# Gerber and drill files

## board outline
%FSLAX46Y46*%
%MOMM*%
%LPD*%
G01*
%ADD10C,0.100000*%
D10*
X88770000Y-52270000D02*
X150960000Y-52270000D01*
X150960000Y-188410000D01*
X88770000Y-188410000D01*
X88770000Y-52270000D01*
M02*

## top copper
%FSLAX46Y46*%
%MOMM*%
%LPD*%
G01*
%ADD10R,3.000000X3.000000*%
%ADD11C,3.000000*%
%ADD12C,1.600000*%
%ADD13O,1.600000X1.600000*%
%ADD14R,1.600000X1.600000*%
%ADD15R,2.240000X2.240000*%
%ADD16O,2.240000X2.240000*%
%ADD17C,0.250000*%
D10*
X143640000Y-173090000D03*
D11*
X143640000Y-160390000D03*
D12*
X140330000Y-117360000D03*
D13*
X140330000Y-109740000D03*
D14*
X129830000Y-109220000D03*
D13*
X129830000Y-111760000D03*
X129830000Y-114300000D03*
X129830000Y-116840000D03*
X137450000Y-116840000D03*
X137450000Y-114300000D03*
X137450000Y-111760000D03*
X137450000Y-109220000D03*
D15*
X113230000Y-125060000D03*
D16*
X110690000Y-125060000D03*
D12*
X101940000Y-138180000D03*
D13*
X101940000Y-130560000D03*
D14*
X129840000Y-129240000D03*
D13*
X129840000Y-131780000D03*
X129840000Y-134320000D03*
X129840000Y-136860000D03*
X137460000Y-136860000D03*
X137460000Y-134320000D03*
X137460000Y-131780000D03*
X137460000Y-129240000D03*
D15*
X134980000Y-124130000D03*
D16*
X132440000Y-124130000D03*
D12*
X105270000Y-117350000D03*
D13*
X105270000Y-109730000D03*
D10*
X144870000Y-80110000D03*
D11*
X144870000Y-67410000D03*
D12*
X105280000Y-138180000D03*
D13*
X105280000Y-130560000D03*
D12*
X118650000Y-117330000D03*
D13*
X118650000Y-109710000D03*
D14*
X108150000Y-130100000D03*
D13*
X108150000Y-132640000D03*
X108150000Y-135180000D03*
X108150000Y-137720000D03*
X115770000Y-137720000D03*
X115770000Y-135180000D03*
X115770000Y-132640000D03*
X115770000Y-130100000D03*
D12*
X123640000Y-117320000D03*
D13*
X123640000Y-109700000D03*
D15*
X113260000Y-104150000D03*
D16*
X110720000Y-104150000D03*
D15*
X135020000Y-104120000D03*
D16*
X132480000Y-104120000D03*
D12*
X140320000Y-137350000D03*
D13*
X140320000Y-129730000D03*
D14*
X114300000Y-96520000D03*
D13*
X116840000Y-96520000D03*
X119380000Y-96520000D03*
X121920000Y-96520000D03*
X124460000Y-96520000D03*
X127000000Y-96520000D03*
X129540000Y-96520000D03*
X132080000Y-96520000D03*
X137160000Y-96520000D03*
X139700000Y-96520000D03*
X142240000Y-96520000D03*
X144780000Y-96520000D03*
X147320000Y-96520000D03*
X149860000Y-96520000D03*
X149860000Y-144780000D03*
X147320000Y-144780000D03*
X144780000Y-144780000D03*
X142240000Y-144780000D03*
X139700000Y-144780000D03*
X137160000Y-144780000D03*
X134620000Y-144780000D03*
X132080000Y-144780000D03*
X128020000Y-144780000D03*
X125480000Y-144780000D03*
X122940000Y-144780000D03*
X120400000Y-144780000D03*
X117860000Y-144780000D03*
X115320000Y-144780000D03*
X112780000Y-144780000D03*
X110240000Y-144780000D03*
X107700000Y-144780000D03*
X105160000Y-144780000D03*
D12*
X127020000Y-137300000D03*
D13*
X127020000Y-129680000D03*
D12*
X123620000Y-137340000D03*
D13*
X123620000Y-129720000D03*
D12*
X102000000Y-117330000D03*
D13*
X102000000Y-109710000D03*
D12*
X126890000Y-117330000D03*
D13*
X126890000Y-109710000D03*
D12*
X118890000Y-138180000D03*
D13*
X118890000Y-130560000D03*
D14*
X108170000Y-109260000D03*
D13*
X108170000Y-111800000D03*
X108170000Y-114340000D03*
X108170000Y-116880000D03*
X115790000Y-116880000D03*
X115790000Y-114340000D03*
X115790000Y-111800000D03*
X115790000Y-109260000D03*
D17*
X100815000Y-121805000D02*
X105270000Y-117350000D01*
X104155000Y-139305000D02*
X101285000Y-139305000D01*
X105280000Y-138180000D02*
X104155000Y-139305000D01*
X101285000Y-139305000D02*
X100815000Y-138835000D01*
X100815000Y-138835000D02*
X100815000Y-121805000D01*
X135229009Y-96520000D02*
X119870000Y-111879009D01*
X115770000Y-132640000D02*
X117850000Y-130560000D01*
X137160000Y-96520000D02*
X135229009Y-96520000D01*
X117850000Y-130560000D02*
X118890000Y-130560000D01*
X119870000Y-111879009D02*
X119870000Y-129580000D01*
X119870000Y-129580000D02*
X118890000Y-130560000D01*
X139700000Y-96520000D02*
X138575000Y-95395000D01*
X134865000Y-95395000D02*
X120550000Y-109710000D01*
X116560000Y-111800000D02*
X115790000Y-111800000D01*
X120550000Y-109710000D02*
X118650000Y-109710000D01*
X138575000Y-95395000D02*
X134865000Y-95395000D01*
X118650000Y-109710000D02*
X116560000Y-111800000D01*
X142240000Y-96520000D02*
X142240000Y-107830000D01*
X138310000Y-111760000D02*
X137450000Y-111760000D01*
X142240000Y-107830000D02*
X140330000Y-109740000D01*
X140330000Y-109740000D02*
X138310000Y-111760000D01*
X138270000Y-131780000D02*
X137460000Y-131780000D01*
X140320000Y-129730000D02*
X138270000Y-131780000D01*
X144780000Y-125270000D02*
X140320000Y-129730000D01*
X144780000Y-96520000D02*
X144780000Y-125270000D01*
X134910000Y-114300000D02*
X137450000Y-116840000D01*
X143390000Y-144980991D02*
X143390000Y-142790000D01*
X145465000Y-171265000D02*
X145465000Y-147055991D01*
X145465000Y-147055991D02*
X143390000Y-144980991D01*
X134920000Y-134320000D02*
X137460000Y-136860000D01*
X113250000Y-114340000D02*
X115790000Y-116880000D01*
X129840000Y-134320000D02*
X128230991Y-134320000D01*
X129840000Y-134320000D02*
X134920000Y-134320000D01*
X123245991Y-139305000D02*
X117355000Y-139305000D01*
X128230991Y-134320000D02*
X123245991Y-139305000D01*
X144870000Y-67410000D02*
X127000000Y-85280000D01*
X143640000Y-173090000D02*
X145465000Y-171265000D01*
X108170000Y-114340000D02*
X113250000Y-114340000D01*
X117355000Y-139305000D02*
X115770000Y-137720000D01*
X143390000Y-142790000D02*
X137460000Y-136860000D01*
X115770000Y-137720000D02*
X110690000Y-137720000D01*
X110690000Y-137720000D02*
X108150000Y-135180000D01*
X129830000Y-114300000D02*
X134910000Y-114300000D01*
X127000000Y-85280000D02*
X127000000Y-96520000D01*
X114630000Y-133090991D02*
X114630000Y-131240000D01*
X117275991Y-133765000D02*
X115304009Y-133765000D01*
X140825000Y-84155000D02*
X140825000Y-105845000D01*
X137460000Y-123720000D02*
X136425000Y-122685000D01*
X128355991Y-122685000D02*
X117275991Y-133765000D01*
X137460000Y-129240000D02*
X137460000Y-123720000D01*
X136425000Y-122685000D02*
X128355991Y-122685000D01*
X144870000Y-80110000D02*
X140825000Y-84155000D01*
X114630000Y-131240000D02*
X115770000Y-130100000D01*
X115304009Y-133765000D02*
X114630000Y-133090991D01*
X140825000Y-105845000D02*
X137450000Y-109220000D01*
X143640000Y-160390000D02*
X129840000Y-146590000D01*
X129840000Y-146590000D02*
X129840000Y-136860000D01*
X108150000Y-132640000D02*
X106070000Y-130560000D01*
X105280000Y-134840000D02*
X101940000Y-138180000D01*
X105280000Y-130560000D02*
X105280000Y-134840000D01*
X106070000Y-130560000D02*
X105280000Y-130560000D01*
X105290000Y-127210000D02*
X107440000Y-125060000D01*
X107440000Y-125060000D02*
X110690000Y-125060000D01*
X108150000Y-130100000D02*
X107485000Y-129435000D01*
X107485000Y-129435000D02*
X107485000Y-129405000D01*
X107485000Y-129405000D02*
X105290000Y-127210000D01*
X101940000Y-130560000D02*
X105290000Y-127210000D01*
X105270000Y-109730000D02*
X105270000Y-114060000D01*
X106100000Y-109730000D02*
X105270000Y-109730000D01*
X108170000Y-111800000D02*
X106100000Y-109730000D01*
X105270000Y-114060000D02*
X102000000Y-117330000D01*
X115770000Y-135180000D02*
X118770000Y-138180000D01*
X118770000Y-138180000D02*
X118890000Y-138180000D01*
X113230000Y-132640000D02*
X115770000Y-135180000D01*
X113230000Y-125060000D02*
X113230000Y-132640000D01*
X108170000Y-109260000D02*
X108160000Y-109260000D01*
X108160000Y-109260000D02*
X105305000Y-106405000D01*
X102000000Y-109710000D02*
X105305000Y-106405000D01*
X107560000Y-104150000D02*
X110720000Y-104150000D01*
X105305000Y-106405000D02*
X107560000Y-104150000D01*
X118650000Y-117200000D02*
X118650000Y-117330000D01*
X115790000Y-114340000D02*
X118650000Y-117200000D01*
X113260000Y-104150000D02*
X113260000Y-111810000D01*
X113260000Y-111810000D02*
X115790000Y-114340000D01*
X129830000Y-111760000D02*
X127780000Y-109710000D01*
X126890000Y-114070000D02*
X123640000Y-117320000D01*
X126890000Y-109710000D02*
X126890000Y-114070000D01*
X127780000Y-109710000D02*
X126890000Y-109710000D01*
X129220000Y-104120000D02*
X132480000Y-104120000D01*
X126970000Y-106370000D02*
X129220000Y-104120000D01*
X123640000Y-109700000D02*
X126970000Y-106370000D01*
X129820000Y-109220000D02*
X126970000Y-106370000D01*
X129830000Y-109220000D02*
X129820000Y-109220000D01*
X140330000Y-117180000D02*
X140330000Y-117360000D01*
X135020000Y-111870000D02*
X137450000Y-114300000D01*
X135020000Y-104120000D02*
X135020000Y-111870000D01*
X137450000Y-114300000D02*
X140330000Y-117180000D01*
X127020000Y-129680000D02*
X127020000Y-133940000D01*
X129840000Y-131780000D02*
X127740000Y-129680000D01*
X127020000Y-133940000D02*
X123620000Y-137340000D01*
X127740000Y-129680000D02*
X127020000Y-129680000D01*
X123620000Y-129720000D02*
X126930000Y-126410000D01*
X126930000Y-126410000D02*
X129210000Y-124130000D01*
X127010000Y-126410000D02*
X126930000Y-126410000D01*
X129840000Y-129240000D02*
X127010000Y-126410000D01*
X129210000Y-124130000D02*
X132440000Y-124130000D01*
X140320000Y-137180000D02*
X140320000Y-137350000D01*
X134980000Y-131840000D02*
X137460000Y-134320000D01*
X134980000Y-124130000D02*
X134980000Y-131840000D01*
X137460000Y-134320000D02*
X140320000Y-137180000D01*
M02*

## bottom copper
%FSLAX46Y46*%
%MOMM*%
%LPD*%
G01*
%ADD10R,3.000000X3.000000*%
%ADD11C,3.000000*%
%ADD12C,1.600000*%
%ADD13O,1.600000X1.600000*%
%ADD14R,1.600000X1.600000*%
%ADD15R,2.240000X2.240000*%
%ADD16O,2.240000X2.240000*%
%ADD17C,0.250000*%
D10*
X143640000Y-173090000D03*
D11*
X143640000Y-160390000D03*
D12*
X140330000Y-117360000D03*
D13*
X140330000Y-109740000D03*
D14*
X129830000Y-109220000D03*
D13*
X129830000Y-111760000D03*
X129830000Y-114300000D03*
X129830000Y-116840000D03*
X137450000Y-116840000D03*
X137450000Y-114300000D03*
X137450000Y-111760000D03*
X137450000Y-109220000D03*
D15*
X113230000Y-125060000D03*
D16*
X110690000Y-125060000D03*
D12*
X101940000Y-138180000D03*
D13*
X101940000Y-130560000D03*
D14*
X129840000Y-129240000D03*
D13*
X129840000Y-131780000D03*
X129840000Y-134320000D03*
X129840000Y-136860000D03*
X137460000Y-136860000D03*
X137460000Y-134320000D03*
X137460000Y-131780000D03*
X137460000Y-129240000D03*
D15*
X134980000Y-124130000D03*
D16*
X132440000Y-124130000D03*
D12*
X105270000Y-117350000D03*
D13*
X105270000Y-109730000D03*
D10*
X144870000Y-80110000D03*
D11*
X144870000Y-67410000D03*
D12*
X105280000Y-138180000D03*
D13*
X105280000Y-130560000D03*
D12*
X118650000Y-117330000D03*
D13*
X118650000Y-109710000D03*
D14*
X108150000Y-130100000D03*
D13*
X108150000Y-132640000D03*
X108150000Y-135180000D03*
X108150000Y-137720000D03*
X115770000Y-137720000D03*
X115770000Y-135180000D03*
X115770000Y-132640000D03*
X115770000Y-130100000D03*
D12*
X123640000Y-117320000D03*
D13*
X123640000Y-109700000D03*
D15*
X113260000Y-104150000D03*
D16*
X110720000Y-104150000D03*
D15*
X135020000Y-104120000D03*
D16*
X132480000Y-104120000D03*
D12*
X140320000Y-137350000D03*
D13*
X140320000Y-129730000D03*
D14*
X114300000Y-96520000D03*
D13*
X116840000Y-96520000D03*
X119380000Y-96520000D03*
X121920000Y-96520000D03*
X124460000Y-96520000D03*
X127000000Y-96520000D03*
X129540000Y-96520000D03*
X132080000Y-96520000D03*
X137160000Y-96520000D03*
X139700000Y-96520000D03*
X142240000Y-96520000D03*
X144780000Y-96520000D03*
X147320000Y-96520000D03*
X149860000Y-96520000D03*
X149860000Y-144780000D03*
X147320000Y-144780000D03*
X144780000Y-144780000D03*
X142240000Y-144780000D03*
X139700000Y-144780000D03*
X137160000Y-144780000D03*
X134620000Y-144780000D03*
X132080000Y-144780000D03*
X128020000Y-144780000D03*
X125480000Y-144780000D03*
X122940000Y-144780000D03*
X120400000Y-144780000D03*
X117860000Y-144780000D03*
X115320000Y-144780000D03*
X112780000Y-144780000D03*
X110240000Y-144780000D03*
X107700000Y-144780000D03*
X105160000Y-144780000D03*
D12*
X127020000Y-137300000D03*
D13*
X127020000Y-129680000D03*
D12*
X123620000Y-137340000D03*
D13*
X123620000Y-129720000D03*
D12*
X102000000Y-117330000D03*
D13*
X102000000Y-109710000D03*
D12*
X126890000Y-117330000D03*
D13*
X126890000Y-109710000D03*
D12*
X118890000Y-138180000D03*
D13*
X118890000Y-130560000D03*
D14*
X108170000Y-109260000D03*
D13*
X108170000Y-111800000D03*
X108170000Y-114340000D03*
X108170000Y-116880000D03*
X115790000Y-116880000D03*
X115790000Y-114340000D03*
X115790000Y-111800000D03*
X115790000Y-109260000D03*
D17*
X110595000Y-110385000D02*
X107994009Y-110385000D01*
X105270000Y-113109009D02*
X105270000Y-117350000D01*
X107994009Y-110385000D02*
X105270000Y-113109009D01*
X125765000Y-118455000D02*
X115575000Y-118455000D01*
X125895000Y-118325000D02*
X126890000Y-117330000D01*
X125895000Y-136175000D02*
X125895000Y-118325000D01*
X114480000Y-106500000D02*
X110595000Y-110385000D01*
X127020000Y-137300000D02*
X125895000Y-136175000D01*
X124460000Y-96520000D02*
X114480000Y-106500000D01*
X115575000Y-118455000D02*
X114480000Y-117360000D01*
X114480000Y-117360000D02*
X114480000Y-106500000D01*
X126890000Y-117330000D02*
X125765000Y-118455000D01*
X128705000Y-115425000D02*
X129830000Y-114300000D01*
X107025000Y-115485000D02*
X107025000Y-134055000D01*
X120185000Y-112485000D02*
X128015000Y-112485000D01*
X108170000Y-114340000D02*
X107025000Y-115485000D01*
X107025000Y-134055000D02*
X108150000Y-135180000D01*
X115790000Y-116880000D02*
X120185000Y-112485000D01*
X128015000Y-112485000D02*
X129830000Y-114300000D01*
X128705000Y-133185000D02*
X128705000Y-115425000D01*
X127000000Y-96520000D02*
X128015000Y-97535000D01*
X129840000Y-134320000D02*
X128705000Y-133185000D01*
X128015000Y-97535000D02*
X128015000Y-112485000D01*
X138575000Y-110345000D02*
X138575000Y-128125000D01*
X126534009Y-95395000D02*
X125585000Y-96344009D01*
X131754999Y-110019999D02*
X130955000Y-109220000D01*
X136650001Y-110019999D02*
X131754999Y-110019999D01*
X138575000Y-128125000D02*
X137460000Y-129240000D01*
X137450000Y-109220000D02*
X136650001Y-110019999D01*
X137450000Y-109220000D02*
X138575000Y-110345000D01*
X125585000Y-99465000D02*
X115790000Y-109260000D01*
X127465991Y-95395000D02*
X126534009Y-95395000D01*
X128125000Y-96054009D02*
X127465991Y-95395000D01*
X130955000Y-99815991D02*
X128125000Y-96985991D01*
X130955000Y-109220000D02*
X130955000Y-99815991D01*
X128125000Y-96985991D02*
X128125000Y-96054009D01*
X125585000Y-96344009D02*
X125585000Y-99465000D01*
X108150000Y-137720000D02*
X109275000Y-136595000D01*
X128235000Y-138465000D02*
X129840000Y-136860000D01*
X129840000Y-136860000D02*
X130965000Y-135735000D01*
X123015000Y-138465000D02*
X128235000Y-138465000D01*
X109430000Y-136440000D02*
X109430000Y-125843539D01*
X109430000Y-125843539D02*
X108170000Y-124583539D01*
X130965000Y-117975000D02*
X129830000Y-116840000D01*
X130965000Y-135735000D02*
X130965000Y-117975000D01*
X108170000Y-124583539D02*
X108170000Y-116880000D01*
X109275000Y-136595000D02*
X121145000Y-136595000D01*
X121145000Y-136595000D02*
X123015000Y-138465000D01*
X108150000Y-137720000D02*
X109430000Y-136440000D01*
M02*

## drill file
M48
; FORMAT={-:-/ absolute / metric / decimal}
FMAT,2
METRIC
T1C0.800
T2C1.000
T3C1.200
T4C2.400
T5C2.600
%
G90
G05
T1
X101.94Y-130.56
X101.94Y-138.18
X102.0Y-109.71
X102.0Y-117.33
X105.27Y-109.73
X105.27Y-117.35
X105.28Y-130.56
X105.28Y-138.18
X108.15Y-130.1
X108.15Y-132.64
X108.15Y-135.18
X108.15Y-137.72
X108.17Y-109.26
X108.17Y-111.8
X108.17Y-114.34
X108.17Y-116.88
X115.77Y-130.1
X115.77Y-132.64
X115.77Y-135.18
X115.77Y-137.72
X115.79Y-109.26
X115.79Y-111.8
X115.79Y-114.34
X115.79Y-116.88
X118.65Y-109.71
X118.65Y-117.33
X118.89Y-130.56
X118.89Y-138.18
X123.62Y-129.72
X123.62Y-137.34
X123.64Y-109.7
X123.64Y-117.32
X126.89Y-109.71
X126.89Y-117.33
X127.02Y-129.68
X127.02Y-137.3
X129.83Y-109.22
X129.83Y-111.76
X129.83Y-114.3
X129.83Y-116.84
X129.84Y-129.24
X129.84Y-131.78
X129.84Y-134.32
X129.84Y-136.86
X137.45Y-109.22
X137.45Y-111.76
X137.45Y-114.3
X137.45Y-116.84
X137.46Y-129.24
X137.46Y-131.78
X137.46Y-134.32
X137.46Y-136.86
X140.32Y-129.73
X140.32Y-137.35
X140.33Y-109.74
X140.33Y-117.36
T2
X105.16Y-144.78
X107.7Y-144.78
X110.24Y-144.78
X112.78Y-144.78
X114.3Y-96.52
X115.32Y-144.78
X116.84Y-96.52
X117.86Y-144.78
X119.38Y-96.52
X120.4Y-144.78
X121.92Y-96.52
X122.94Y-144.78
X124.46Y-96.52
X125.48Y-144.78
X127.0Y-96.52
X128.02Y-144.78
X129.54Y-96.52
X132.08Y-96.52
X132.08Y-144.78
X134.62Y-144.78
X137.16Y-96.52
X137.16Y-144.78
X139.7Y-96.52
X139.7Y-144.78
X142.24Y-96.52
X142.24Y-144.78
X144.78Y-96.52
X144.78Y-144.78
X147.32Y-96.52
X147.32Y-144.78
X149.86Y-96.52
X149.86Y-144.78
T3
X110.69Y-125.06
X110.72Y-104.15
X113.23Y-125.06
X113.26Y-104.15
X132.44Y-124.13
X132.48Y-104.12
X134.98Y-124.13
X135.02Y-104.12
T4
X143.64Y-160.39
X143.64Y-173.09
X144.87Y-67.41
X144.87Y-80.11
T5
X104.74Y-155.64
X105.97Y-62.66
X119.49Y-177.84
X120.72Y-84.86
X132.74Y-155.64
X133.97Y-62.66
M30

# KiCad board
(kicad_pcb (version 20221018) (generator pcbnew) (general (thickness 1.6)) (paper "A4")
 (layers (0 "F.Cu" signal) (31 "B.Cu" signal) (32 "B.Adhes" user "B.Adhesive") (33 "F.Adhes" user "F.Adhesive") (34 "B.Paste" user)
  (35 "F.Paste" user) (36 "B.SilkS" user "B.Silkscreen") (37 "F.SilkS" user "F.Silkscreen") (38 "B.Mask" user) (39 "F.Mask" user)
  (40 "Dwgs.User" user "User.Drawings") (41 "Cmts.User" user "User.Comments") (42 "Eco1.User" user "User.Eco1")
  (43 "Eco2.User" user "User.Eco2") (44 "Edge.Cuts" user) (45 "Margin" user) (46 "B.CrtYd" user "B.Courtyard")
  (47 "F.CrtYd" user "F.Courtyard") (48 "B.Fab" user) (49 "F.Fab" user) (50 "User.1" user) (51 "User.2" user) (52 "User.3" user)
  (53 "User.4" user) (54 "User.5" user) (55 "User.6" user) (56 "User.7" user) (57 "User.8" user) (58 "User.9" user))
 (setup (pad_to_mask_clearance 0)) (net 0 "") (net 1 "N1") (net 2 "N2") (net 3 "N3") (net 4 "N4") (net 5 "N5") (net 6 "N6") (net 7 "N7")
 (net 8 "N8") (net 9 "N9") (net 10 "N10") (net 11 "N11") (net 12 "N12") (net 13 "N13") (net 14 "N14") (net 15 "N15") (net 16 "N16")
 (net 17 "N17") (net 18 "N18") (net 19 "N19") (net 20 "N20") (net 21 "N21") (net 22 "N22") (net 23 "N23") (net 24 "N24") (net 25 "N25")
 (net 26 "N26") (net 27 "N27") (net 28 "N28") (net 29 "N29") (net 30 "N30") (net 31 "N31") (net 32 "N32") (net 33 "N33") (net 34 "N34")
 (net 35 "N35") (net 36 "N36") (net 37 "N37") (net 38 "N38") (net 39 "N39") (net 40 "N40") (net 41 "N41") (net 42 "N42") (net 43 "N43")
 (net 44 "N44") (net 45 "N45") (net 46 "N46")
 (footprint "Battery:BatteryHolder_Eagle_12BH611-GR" (layer "F.Cu") (at 143.64 173.09)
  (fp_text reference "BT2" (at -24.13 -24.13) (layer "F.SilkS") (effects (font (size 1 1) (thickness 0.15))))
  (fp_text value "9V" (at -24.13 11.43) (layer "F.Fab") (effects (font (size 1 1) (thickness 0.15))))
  (pad "" np_thru_hole circle (at -38.9 -17.45) (size 2.6 2.6) (drill 2.6) (layers "*.Cu" "*.Mask"))
  (pad "" np_thru_hole circle (at -24.15 4.75) (size 2.6 2.6) (drill 2.6) (layers "*.Cu" "*.Mask"))
  (pad "" np_thru_hole circle (at -10.9 -17.45) (size 2.6 2.6) (drill 2.6) (layers "*.Cu" "*.Mask"))
  (pad "1" thru_hole rect (at 0 0) (size 3 3) (drill 2.4) (layers "*.Cu" "*.Mask") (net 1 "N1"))
  (pad "2" thru_hole circle (at 0 -12.7) (size 3 3) (drill 2.4) (layers "*.Cu" "*.Mask") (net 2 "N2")))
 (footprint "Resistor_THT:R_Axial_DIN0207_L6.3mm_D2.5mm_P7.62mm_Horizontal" (layer "F.Cu") (at 140.33 117.36 90)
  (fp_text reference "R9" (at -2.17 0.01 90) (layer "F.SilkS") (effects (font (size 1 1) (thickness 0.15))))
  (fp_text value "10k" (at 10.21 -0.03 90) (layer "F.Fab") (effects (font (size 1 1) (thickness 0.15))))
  (pad "1" thru_hole circle (at 0 0 90) (size 1.6 1.6) (drill 0.8) (layers "*.Cu" "*.Mask") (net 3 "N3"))
  (pad "2" thru_hole oval (at 7.62 0 90) (size 1.6 1.6) (drill 0.8) (layers "*.Cu" "*.Mask") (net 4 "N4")))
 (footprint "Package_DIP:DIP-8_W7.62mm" (layer "F.Cu") (at 129.83 109.22)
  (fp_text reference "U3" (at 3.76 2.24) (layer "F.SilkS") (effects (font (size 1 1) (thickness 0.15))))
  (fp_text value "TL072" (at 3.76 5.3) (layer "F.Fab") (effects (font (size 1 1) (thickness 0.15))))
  (pad "1" thru_hole rect (at 0 0) (size 1.6 1.6) (drill 0.8) (layers "*.Cu" "*.Mask") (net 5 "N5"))
  (pad "2" thru_hole oval (at 0 2.54) (size 1.6 1.6) (drill 0.8) (layers "*.Cu" "*.Mask") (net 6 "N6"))
  (pad "3" thru_hole oval (at 0 5.08) (size 1.6 1.6) (drill 0.8) (layers "*.Cu" "*.Mask") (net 1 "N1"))
  (pad "4" thru_hole oval (at 0 7.62) (size 1.6 1.6) (drill 0.8) (layers "*.Cu" "*.Mask") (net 2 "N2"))
  (pad "5" thru_hole oval (at 7.62 7.62) (size 1.6 1.6) (drill 0.8) (layers "*.Cu" "*.Mask") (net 1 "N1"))
  (pad "6" thru_hole oval (at 7.62 5.08) (size 1.6 1.6) (drill 0.8) (layers "*.Cu" "*.Mask") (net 3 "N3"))
  (pad "7" thru_hole oval (at 7.62 2.54) (size 1.6 1.6) (drill 0.8) (layers "*.Cu" "*.Mask") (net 4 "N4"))
  (pad "8" thru_hole oval (at 7.62 0) (size 1.6 1.6) (drill 0.8) (layers "*.Cu" "*.Mask") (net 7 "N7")))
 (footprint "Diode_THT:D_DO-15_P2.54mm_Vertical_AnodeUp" (layer "F.Cu") (at 113.23 125.06 180)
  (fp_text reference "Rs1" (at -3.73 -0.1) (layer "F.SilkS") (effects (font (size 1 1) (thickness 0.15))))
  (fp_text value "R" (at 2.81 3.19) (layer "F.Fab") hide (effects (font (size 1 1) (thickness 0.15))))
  (pad "1" thru_hole rect (at 0 0 180) (size 2.24 2.24) (drill 1.2) (layers "*.Cu" "*.Mask") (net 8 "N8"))
  (pad "2" thru_hole oval (at 2.54 0 180) (size 2.24 2.24) (drill 1.2) (layers "*.Cu" "*.Mask") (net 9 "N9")))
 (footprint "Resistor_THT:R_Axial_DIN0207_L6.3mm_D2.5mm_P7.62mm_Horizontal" (layer "F.Cu") (at 101.94 138.18 90)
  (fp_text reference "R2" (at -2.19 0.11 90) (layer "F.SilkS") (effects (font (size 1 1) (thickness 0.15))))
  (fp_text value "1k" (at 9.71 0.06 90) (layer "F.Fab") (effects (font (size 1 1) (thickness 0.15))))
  (pad "1" thru_hole circle (at 0 0 90) (size 1.6 1.6) (drill 0.8) (layers "*.Cu" "*.Mask") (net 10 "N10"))
  (pad "2" thru_hole oval (at 7.62 0 90) (size 1.6 1.6) (drill 0.8) (layers "*.Cu" "*.Mask") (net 9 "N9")))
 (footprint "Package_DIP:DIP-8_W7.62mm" (layer "F.Cu") (at 129.84 129.24)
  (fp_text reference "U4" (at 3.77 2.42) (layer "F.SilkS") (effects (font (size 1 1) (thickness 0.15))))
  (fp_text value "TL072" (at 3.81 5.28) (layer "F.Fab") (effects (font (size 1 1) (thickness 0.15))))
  (pad "1" thru_hole rect (at 0 0) (size 1.6 1.6) (drill 0.8) (layers "*.Cu" "*.Mask") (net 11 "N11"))
  (pad "2" thru_hole oval (at 0 2.54) (size 1.6 1.6) (drill 0.8) (layers "*.Cu" "*.Mask") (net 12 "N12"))
  (pad "3" thru_hole oval (at 0 5.08) (size 1.6 1.6) (drill 0.8) (layers "*.Cu" "*.Mask") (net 1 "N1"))
  (pad "4" thru_hole oval (at 0 7.62) (size 1.6 1.6) (drill 0.8) (layers "*.Cu" "*.Mask") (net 2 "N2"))
  (pad "5" thru_hole oval (at 7.62 7.62) (size 1.6 1.6) (drill 0.8) (layers "*.Cu" "*.Mask") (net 1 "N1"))
  (pad "6" thru_hole oval (at 7.62 5.08) (size 1.6 1.6) (drill 0.8) (layers "*.Cu" "*.Mask") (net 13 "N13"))
  (pad "7" thru_hole oval (at 7.62 2.54) (size 1.6 1.6) (drill 0.8) (layers "*.Cu" "*.Mask") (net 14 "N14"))
  (pad "8" thru_hole oval (at 7.62 0) (size 1.6 1.6) (drill 0.8) (layers "*.Cu" "*.Mask") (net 7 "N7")))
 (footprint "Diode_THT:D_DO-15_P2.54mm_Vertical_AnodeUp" (layer "F.Cu") (at 134.98 124.13 180)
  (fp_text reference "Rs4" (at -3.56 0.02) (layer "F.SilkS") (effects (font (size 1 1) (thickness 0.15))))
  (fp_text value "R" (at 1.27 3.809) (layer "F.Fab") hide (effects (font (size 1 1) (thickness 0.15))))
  (pad "1" thru_hole rect (at 0 0 180) (size 2.24 2.24) (drill 1.2) (layers "*.Cu" "*.Mask") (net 13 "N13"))
  (pad "2" thru_hole oval (at 2.54 0 180) (size 2.24 2.24) (drill 1.2) (layers "*.Cu" "*.Mask") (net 11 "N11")))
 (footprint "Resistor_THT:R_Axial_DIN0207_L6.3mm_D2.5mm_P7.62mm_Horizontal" (layer "F.Cu") (at 105.27 117.35 90)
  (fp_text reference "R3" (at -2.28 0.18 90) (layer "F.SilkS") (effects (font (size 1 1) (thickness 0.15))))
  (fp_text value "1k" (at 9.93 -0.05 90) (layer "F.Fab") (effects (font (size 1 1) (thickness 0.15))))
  (pad "1" thru_hole circle (at 0 0 90) (size 1.6 1.6) (drill 0.8) (layers "*.Cu" "*.Mask") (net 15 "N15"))
  (pad "2" thru_hole oval (at 7.62 0 90) (size 1.6 1.6) (drill 0.8) (layers "*.Cu" "*.Mask") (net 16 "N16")))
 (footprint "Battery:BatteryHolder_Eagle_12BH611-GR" (layer "F.Cu") (at 144.87 80.11)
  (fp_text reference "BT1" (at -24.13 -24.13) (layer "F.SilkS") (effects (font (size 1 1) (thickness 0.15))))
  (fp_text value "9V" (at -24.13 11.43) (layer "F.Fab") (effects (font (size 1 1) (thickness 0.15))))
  (pad "" np_thru_hole circle (at -38.9 -17.45) (size 2.6 2.6) (drill 2.6) (layers "*.Cu" "*.Mask"))
  (pad "" np_thru_hole circle (at -24.15 4.75) (size 2.6 2.6) (drill 2.6) (layers "*.Cu" "*.Mask"))
  (pad "" np_thru_hole circle (at -10.9 -17.45) (size 2.6 2.6) (drill 2.6) (layers "*.Cu" "*.Mask"))
  (pad "1" thru_hole rect (at 0 0) (size 3 3) (drill 2.4) (layers "*.Cu" "*.Mask") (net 7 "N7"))
  (pad "2" thru_hole circle (at 0 -12.7) (size 3 3) (drill 2.4) (layers "*.Cu" "*.Mask") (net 1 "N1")))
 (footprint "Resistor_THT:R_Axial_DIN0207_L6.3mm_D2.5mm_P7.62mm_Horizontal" (layer "F.Cu") (at 105.28 138.18 90)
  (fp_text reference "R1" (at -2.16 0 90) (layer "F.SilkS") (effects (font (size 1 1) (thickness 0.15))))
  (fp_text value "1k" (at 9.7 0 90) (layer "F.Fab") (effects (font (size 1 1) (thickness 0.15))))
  (pad "1" thru_hole circle (at 0 0 90) (size 1.6 1.6) (drill 0.8) (layers "*.Cu" "*.Mask") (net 15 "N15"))
  (pad "2" thru_hole oval (at 7.62 0 90) (size 1.6 1.6) (drill 0.8) (layers "*.Cu" "*.Mask") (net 10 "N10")))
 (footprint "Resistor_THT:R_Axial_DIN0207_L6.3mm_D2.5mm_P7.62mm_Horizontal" (layer "F.Cu") (at 118.65 117.33 90)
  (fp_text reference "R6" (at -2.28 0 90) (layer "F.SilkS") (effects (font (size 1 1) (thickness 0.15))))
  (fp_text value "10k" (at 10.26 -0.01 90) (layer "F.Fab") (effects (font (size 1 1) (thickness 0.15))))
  (pad "1" thru_hole circle (at 0 0 90) (size 1.6 1.6) (drill 0.8) (layers "*.Cu" "*.Mask") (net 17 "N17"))
  (pad "2" thru_hole oval (at 7.62 0 90) (size 1.6 1.6) (drill 0.8) (layers "*.Cu" "*.Mask") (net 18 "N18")))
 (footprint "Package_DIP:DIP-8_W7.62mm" (layer "F.Cu") (at 108.15 130.1)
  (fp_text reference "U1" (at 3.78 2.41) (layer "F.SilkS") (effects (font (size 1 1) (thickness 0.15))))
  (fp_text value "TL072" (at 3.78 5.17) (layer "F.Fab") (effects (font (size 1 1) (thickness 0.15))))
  (pad "1" thru_hole rect (at 0 0) (size 1.6 1.6) (drill 0.8) (layers "*.Cu" "*.Mask") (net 9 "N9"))
  (pad "2" thru_hole oval (at 0 2.54) (size 1.6 1.6) (drill 0.8) (layers "*.Cu" "*.Mask") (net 10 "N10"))
  (pad "3" thru_hole oval (at 0 5.08) (size 1.6 1.6) (drill 0.8) (layers "*.Cu" "*.Mask") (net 1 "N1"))
  (pad "4" thru_hole oval (at 0 7.62) (size 1.6 1.6) (drill 0.8) (layers "*.Cu" "*.Mask") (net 2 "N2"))
  (pad "5" thru_hole oval (at 7.62 7.62) (size 1.6 1.6) (drill 0.8) (layers "*.Cu" "*.Mask") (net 1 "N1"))
  (pad "6" thru_hole oval (at 7.62 5.08) (size 1.6 1.6) (drill 0.8) (layers "*.Cu" "*.Mask") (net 8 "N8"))
  (pad "7" thru_hole oval (at 7.62 2.54) (size 1.6 1.6) (drill 0.8) (layers "*.Cu" "*.Mask") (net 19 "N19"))
  (pad "8" thru_hole oval (at 7.62 0) (size 1.6 1.6) (drill 0.8) (layers "*.Cu" "*.Mask") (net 7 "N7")))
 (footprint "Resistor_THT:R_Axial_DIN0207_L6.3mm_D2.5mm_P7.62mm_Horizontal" (layer "F.Cu") (at 123.64 117.32 90)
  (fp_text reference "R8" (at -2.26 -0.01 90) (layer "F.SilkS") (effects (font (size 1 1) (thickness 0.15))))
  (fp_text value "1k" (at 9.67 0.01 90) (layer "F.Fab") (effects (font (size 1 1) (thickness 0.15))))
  (pad "1" thru_hole circle (at 0 0 90) (size 1.6 1.6) (drill 0.8) (layers "*.Cu" "*.Mask") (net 6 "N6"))
  (pad "2" thru_hole oval (at 7.62 0 90) (size 1.6 1.6) (drill 0.8) (layers "*.Cu" "*.Mask") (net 5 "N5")))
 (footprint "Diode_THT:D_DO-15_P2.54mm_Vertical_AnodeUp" (layer "F.Cu") (at 113.26 104.15 180)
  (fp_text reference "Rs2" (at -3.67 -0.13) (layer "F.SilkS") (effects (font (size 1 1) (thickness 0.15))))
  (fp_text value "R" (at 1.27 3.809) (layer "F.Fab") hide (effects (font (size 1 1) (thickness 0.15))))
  (pad "1" thru_hole rect (at 0 0 180) (size 2.24 2.24) (drill 1.2) (layers "*.Cu" "*.Mask") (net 17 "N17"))
  (pad "2" thru_hole oval (at 2.54 0 180) (size 2.24 2.24) (drill 1.2) (layers "*.Cu" "*.Mask") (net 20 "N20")))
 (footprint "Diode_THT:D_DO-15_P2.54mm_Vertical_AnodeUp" (layer "F.Cu") (at 135.02 104.12 180)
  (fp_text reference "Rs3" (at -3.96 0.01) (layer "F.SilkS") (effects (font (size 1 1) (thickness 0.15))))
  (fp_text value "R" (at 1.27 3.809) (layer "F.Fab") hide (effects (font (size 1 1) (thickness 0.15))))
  (pad "1" thru_hole rect (at 0 0 180) (size 2.24 2.24) (drill 1.2) (layers "*.Cu" "*.Mask") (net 3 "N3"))
  (pad "2" thru_hole oval (at 2.54 0 180) (size 2.24 2.24) (drill 1.2) (layers "*.Cu" "*.Mask") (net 5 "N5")))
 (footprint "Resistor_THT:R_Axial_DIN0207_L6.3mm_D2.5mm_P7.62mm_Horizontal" (layer "F.Cu") (at 140.32 137.35 90)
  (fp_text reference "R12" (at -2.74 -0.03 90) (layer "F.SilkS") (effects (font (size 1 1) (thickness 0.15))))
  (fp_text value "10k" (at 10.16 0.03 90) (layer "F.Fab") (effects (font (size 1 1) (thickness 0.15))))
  (pad "1" thru_hole circle (at 0 0 90) (size 1.6 1.6) (drill 0.8) (layers "*.Cu" "*.Mask") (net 13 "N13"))
  (pad "2" thru_hole oval (at 7.62 0 90) (size 1.6 1.6) (drill 0.8) (layers "*.Cu" "*.Mask") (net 14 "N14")))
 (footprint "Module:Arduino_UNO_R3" (layer "F.Cu") (at 114.3 96.52)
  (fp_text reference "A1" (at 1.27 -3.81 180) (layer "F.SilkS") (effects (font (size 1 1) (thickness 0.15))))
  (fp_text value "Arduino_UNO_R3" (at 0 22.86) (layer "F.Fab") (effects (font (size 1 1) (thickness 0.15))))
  (pad "1" thru_hole rect (at 0 0 90) (size 1.6 1.6) (drill 1) (layers "*.Cu" "*.Mask") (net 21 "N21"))
  (pad "2" thru_hole oval (at 2.54 0 90) (size 1.6 1.6) (drill 1) (layers "*.Cu" "*.Mask") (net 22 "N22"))
  (pad "3" thru_hole oval (at 5.08 0 90) (size 1.6 1.6) (drill 1) (layers "*.Cu" "*.Mask") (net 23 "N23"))
  (pad "4" thru_hole oval (at 7.62 0 90) (size 1.6 1.6) (drill 1) (layers "*.Cu" "*.Mask") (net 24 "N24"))
  (pad "5" thru_hole oval (at 10.16 0 90) (size 1.6 1.6) (drill 1) (layers "*.Cu" "*.Mask") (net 15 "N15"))
  (pad "6" thru_hole oval (at 12.7 0 90) (size 1.6 1.6) (drill 1) (layers "*.Cu" "*.Mask") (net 1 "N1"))
  (pad "7" thru_hole oval (at 15.24 0 90) (size 1.6 1.6) (drill 1) (layers "*.Cu" "*.Mask") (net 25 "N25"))
  (pad "8" thru_hole oval (at 17.78 0 90) (size 1.6 1.6) (drill 1) (layers "*.Cu" "*.Mask") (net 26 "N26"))
  (pad "9" thru_hole oval (at 22.86 0 90) (size 1.6 1.6) (drill 1) (layers "*.Cu" "*.Mask") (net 19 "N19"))
  (pad "10" thru_hole oval (at 25.4 0 90) (size 1.6 1.6) (drill 1) (layers "*.Cu" "*.Mask") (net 18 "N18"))
  (pad "11" thru_hole oval (at 27.94 0 90) (size 1.6 1.6) (drill 1) (layers "*.Cu" "*.Mask") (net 4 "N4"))
  (pad "12" thru_hole oval (at 30.48 0 90) (size 1.6 1.6) (drill 1) (layers "*.Cu" "*.Mask") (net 14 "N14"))
  (pad "13" thru_hole oval (at 33.02 0 90) (size 1.6 1.6) (drill 1) (layers "*.Cu" "*.Mask") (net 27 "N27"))
  (pad "14" thru_hole oval (at 35.56 0 90) (size 1.6 1.6) (drill 1) (layers "*.Cu" "*.Mask") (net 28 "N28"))
  (pad "15" thru_hole oval (at 35.56 48.26 90) (size 1.6 1.6) (drill 1) (layers "*.Cu" "*.Mask") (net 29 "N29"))
  (pad "16" thru_hole oval (at 33.02 48.26 90) (size 1.6 1.6) (drill 1) (layers "*.Cu" "*.Mask") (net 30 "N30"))
  (pad "17" thru_hole oval (at 30.48 48.26 90) (size 1.6 1.6) (drill 1) (layers "*.Cu" "*.Mask") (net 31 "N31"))
  (pad "18" thru_hole oval (at 27.94 48.26 90) (size 1.6 1.6) (drill 1) (layers "*.Cu" "*.Mask") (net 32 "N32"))
  (pad "19" thru_hole oval (at 25.4 48.26 90) (size 1.6 1.6) (drill 1) (layers "*.Cu" "*.Mask") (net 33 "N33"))
  (pad "20" thru_hole oval (at 22.86 48.26 90) (size 1.6 1.6) (drill 1) (layers "*.Cu" "*.Mask") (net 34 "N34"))
  (pad "21" thru_hole oval (at 20.32 48.26 90) (size 1.6 1.6) (drill 1) (layers "*.Cu" "*.Mask") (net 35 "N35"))
  (pad "22" thru_hole oval (at 17.78 48.26 90) (size 1.6 1.6) (drill 1) (layers "*.Cu" "*.Mask") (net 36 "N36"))
  (pad "23" thru_hole oval (at 13.72 48.26 90) (size 1.6 1.6) (drill 1) (layers "*.Cu" "*.Mask") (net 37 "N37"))
  (pad "24" thru_hole oval (at 11.18 48.26 90) (size 1.6 1.6) (drill 1) (layers "*.Cu" "*.Mask") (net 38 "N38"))
  (pad "25" thru_hole oval (at 8.64 48.26 90) (size 1.6 1.6) (drill 1) (layers "*.Cu" "*.Mask") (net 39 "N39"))
  (pad "26" thru_hole oval (at 6.1 48.26 90) (size 1.6 1.6) (drill 1) (layers "*.Cu" "*.Mask") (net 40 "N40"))
  (pad "27" thru_hole oval (at 3.56 48.26 90) (size 1.6 1.6) (drill 1) (layers "*.Cu" "*.Mask") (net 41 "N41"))
  (pad "28" thru_hole oval (at 1.02 48.26 90) (size 1.6 1.6) (drill 1) (layers "*.Cu" "*.Mask") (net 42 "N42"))
  (pad "29" thru_hole oval (at -1.52 48.26 90) (size 1.6 1.6) (drill 1) (layers "*.Cu" "*.Mask") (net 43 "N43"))
  (pad "30" thru_hole oval (at -4.06 48.26 90) (size 1.6 1.6) (drill 1) (layers "*.Cu" "*.Mask") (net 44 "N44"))
  (pad "31" thru_hole oval (at -6.6 48.26 90) (size 1.6 1.6) (drill 1) (layers "*.Cu" "*.Mask") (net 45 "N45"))
  (pad "32" thru_hole oval (at -9.14 48.26 90) (size 1.6 1.6) (drill 1) (layers "*.Cu" "*.Mask") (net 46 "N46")))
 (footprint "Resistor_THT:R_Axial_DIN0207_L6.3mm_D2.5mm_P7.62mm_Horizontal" (layer "F.Cu") (at 127.02 137.3 90)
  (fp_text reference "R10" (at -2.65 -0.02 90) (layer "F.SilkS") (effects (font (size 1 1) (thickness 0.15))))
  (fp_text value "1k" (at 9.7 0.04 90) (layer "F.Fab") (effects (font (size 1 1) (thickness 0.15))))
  (pad "1" thru_hole circle (at 0 0 90) (size 1.6 1.6) (drill 0.8) (layers "*.Cu" "*.Mask") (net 15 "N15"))
  (pad "2" thru_hole oval (at 7.62 0 90) (size 1.6 1.6) (drill 0.8) (layers "*.Cu" "*.Mask") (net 12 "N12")))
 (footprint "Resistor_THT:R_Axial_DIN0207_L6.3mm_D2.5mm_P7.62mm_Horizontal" (layer "F.Cu") (at 123.62 137.34 90)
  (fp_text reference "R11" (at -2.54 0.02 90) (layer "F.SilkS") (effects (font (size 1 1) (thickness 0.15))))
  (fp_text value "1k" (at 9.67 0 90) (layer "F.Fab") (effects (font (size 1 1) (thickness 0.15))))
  (pad "1" thru_hole circle (at 0 0 90) (size 1.6 1.6) (drill 0.8) (layers "*.Cu" "*.Mask") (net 12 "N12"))
  (pad "2" thru_hole oval (at 7.62 0 90) (size 1.6 1.6) (drill 0.8) (layers "*.Cu" "*.Mask") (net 11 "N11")))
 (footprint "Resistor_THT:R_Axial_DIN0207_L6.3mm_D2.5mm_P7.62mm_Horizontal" (layer "F.Cu") (at 102 117.33 90)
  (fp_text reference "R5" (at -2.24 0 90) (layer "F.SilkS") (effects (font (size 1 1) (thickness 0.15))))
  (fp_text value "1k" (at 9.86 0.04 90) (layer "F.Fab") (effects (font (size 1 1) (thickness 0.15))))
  (pad "1" thru_hole circle (at 0 0 90) (size 1.6 1.6) (drill 0.8) (layers "*.Cu" "*.Mask") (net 16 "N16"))
  (pad "2" thru_hole oval (at 7.62 0 90) (size 1.6 1.6) (drill 0.8) (layers "*.Cu" "*.Mask") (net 20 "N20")))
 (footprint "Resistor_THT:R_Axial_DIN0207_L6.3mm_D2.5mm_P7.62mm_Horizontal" (layer "F.Cu") (at 126.89 117.33 90)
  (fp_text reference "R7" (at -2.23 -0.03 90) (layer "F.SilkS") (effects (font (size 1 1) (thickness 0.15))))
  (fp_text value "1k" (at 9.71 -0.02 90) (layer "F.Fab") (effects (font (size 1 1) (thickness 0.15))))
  (pad "1" thru_hole circle (at 0 0 90) (size 1.6 1.6) (drill 0.8) (layers "*.Cu" "*.Mask") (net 15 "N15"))
  (pad "2" thru_hole oval (at 7.62 0 90) (size 1.6 1.6) (drill 0.8) (layers "*.Cu" "*.Mask") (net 6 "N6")))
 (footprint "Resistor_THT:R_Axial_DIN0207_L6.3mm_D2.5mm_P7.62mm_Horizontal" (layer "F.Cu") (at 118.89 138.18 90)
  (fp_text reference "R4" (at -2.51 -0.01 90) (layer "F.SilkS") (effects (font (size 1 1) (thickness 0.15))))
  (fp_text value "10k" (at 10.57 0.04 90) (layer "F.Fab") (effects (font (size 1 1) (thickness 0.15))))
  (pad "1" thru_hole circle (at 0 0 90) (size 1.6 1.6) (drill 0.8) (layers "*.Cu" "*.Mask") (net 8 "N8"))
  (pad "2" thru_hole oval (at 7.62 0 90) (size 1.6 1.6) (drill 0.8) (layers "*.Cu" "*.Mask") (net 19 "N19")))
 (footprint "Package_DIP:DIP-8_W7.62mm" (layer "F.Cu") (at 108.17 109.26)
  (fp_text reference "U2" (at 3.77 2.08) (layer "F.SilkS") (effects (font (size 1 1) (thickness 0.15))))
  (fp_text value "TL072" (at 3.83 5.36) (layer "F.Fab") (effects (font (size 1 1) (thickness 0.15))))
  (pad "1" thru_hole rect (at 0 0) (size 1.6 1.6) (drill 0.8) (layers "*.Cu" "*.Mask") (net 20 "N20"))
  (pad "2" thru_hole oval (at 0 2.54) (size 1.6 1.6) (drill 0.8) (layers "*.Cu" "*.Mask") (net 16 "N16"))
  (pad "3" thru_hole oval (at 0 5.08) (size 1.6 1.6) (drill 0.8) (layers "*.Cu" "*.Mask") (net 1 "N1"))
  (pad "4" thru_hole oval (at 0 7.62) (size 1.6 1.6) (drill 0.8) (layers "*.Cu" "*.Mask") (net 2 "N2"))
  (pad "5" thru_hole oval (at 7.62 7.62) (size 1.6 1.6) (drill 0.8) (layers "*.Cu" "*.Mask") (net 1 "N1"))
  (pad "6" thru_hole oval (at 7.62 5.08) (size 1.6 1.6) (drill 0.8) (layers "*.Cu" "*.Mask") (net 17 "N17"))
  (pad "7" thru_hole oval (at 7.62 2.54) (size 1.6 1.6) (drill 0.8) (layers "*.Cu" "*.Mask") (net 18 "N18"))
  (pad "8" thru_hole oval (at 7.62 0) (size 1.6 1.6) (drill 0.8) (layers "*.Cu" "*.Mask") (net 7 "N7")))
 (gr_rect (start 88.77 52.27) (end 150.96 188.41) (stroke (width 0.1) (type default)) (fill none) (layer "Edge.Cuts"))
 (segment (start 100.815 121.805) (end 105.27 117.35) (width 0.25) (layer "F.Cu") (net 15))
 (segment (start 104.155 139.305) (end 101.285 139.305) (width 0.25) (layer "F.Cu") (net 15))
 (segment (start 105.28 138.18) (end 104.155 139.305) (width 0.25) (layer "F.Cu") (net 15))
 (segment (start 101.285 139.305) (end 100.815 138.835) (width 0.25) (layer "F.Cu") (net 15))
 (segment (start 100.815 138.835) (end 100.815 121.805) (width 0.25) (layer "F.Cu") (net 15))
 (segment (start 110.595 110.385) (end 107.994009 110.385) (width 0.25) (layer "B.Cu") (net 15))
 (segment (start 105.27 113.109009) (end 105.27 117.35) (width 0.25) (layer "B.Cu") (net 15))
 (segment (start 107.994009 110.385) (end 105.27 113.109009) (width 0.25) (layer "B.Cu") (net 15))
 (segment (start 125.765 118.455) (end 115.575 118.455) (width 0.25) (layer "B.Cu") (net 15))
 (segment (start 125.895 118.325) (end 126.89 117.33) (width 0.25) (layer "B.Cu") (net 15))
 (segment (start 125.895 136.175) (end 125.895 118.325) (width 0.25) (layer "B.Cu") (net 15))
 (segment (start 114.48 106.5) (end 110.595 110.385) (width 0.25) (layer "B.Cu") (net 15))
 (segment (start 127.02 137.3) (end 125.895 136.175) (width 0.25) (layer "B.Cu") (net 15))
 (segment (start 124.46 96.52) (end 114.48 106.5) (width 0.25) (layer "B.Cu") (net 15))
 (segment (start 115.575 118.455) (end 114.48 117.36) (width 0.25) (layer "B.Cu") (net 15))
 (segment (start 114.48 117.36) (end 114.48 106.5) (width 0.25) (layer "B.Cu") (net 15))
 (segment (start 126.89 117.33) (end 125.765 118.455) (width 0.25) (layer "B.Cu") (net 15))
 (segment (start 135.229009 96.52) (end 119.87 111.879009) (width 0.25) (layer "F.Cu") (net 19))
 (segment (start 115.77 132.64) (end 117.85 130.56) (width 0.25) (layer "F.Cu") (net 19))
 (segment (start 137.16 96.52) (end 135.229009 96.52) (width 0.25) (layer "F.Cu") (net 19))
 (segment (start 117.85 130.56) (end 118.89 130.56) (width 0.25) (layer "F.Cu") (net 19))
 (segment (start 119.87 111.879009) (end 119.87 129.58) (width 0.25) (layer "F.Cu") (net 19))
 (segment (start 119.87 129.58) (end 118.89 130.56) (width 0.25) (layer "F.Cu") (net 19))
 (segment (start 139.7 96.52) (end 138.575 95.395) (width 0.25) (layer "F.Cu") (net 18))
 (segment (start 134.865 95.395) (end 120.55 109.71) (width 0.25) (layer "F.Cu") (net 18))
 (segment (start 116.56 111.8) (end 115.79 111.8) (width 0.25) (layer "F.Cu") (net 18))
 (segment (start 120.55 109.71) (end 118.65 109.71) (width 0.25) (layer "F.Cu") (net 18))
 (segment (start 138.575 95.395) (end 134.865 95.395) (width 0.25) (layer "F.Cu") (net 18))
 (segment (start 118.65 109.71) (end 116.56 111.8) (width 0.25) (layer "F.Cu") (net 18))
 (segment (start 142.24 96.52) (end 142.24 107.83) (width 0.25) (layer "F.Cu") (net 4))
 (segment (start 138.31 111.76) (end 137.45 111.76) (width 0.25) (layer "F.Cu") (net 4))
 (segment (start 142.24 107.83) (end 140.33 109.74) (width 0.25) (layer "F.Cu") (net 4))
 (segment (start 140.33 109.74) (end 138.31 111.76) (width 0.25) (layer "F.Cu") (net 4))
 (segment (start 138.27 131.78) (end 137.46 131.78) (width 0.25) (layer "F.Cu") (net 14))
 (segment (start 140.32 129.73) (end 138.27 131.78) (width 0.25) (layer "F.Cu") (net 14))
 (segment (start 144.78 125.27) (end 140.32 129.73) (width 0.25) (layer "F.Cu") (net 14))
 (segment (start 144.78 96.52) (end 144.78 125.27) (width 0.25) (layer "F.Cu") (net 14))
 (segment (start 134.91 114.3) (end 137.45 116.84) (width 0.25) (layer "F.Cu") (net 1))
 (segment (start 143.39 144.980991) (end 143.39 142.79) (width 0.25) (layer "F.Cu") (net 1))
 (segment (start 145.465 171.265) (end 145.465 147.055991) (width 0.25) (layer "F.Cu") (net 1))
 (segment (start 145.465 147.055991) (end 143.39 144.980991) (width 0.25) (layer "F.Cu") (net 1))
 (segment (start 134.92 134.32) (end 137.46 136.86) (width 0.25) (layer "F.Cu") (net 1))
 (segment (start 113.25 114.34) (end 115.79 116.88) (width 0.25) (layer "F.Cu") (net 1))
 (segment (start 129.84 134.32) (end 128.230991 134.32) (width 0.25) (layer "F.Cu") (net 1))
 (segment (start 129.84 134.32) (end 134.92 134.32) (width 0.25) (layer "F.Cu") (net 1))
 (segment (start 123.245991 139.305) (end 117.355 139.305) (width 0.25) (layer "F.Cu") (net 1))
 (segment (start 128.230991 134.32) (end 123.245991 139.305) (width 0.25) (layer "F.Cu") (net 1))
 (segment (start 144.87 67.41) (end 127 85.28) (width 0.25) (layer "F.Cu") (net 1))
 (segment (start 143.64 173.09) (end 145.465 171.265) (width 0.25) (layer "F.Cu") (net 1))
 (segment (start 108.17 114.34) (end 113.25 114.34) (width 0.25) (layer "F.Cu") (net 1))
 (segment (start 117.355 139.305) (end 115.77 137.72) (width 0.25) (layer "F.Cu") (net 1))
 (segment (start 143.39 142.79) (end 137.46 136.86) (width 0.25) (layer "F.Cu") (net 1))
 (segment (start 115.77 137.72) (end 110.69 137.72) (width 0.25) (layer "F.Cu") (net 1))
 (segment (start 110.69 137.72) (end 108.15 135.18) (width 0.25) (layer "F.Cu") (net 1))
 (segment (start 129.83 114.3) (end 134.91 114.3) (width 0.25) (layer "F.Cu") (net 1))
 (segment (start 127 85.28) (end 127 96.52) (width 0.25) (layer "F.Cu") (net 1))
 (segment (start 128.705 115.425) (end 129.83 114.3) (width 0.25) (layer "B.Cu") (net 1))
 (segment (start 107.025 115.485) (end 107.025 134.055) (width 0.25) (layer "B.Cu") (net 1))
 (segment (start 120.185 112.485) (end 128.015 112.485) (width 0.25) (layer "B.Cu") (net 1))
 (segment (start 108.17 114.34) (end 107.025 115.485) (width 0.25) (layer "B.Cu") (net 1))
 (segment (start 107.025 134.055) (end 108.15 135.18) (width 0.25) (layer "B.Cu") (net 1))
 (segment (start 115.79 116.88) (end 120.185 112.485) (width 0.25) (layer "B.Cu") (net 1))
 (segment (start 128.015 112.485) (end 129.83 114.3) (width 0.25) (layer "B.Cu") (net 1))
 (segment (start 128.705 133.185) (end 128.705 115.425) (width 0.25) (layer "B.Cu") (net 1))
 (segment (start 127 96.52) (end 128.015 97.535) (width 0.25) (layer "B.Cu") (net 1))
 (segment (start 129.84 134.32) (end 128.705 133.185) (width 0.25) (layer "B.Cu") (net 1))
 (segment (start 128.015 97.535) (end 128.015 112.485) (width 0.25) (layer "B.Cu") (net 1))
 (segment (start 114.63 133.090991) (end 114.63 131.24) (width 0.25) (layer "F.Cu") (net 7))
 (segment (start 117.275991 133.765) (end 115.304009 133.765) (width 0.25) (layer "F.Cu") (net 7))
 (segment (start 140.825 84.155) (end 140.825 105.845) (width 0.25) (layer "F.Cu") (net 7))
 (segment (start 137.46 123.72) (end 136.425 122.685) (width 0.25) (layer "F.Cu") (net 7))
 (segment (start 128.355991 122.685) (end 117.275991 133.765) (width 0.25) (layer "F.Cu") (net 7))
 (segment (start 137.46 129.24) (end 137.46 123.72) (width 0.25) (layer "F.Cu") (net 7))
 (segment (start 136.425 122.685) (end 128.355991 122.685) (width 0.25) (layer "F.Cu") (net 7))
 (segment (start 144.87 80.11) (end 140.825 84.155) (width 0.25) (layer "F.Cu") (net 7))
 (segment (start 114.63 131.24) (end 115.77 130.1) (width 0.25) (layer "F.Cu") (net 7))
 (segment (start 115.304009 133.765) (end 114.63 133.090991) (width 0.25) (layer "F.Cu") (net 7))
 (segment (start 140.825 105.845) (end 137.45 109.22) (width 0.25) (layer "F.Cu") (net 7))
 (segment (start 138.575 110.345) (end 138.575 128.125) (width 0.25) (layer "B.Cu") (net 7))
 (segment (start 126.534009 95.395) (end 125.585 96.344009) (width 0.25) (layer "B.Cu") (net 7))
 (segment (start 131.754999 110.019999) (end 130.955 109.22) (width 0.25) (layer "B.Cu") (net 7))
 (segment (start 136.650001 110.019999) (end 131.754999 110.019999) (width 0.25) (layer "B.Cu") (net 7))
 (segment (start 138.575 128.125) (end 137.46 129.24) (width 0.25) (layer "B.Cu") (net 7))
 (segment (start 137.45 109.22) (end 136.650001 110.019999) (width 0.25) (layer "B.Cu") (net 7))
 (segment (start 137.45 109.22) (end 138.575 110.345) (width 0.25) (layer "B.Cu") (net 7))
 (segment (start 125.585 99.465) (end 115.79 109.26) (width 0.25) (layer "B.Cu") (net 7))
 (segment (start 127.465991 95.395) (end 126.534009 95.395) (width 0.25) (layer "B.Cu") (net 7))
 (segment (start 128.125 96.054009) (end 127.465991 95.395) (width 0.25) (layer "B.Cu") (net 7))
 (segment (start 130.955 99.815991) (end 128.125 96.985991) (width 0.25) (layer "B.Cu") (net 7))
 (segment (start 130.955 109.22) (end 130.955 99.815991) (width 0.25) (layer "B.Cu") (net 7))
 (segment (start 128.125 96.985991) (end 128.125 96.054009) (width 0.25) (layer "B.Cu") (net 7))
 (segment (start 125.585 96.344009) (end 125.585 99.465) (width 0.25) (layer "B.Cu") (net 7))
 (segment (start 143.64 160.39) (end 129.84 146.59) (width 0.25) (layer "F.Cu") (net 2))
 (segment (start 129.84 146.59) (end 129.84 136.86) (width 0.25) (layer "F.Cu") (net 2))
 (segment (start 108.15 137.72) (end 109.275 136.595) (width 0.25) (layer "B.Cu") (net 2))
 (segment (start 128.235 138.465) (end 129.84 136.86) (width 0.25) (layer "B.Cu") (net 2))
 (segment (start 129.84 136.86) (end 130.965 135.735) (width 0.25) (layer "B.Cu") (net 2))
 (segment (start 123.015 138.465) (end 128.235 138.465) (width 0.25) (layer "B.Cu") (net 2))
 (segment (start 109.43 136.44) (end 109.43 125.843539) (width 0.25) (layer "B.Cu") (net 2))
 (segment (start 109.43 125.843539) (end 108.17 124.583539) (width 0.25) (layer "B.Cu") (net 2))
 (segment (start 130.965 117.975) (end 129.83 116.84) (width 0.25) (layer "B.Cu") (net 2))
 (segment (start 130.965 135.735) (end 130.965 117.975) (width 0.25) (layer "B.Cu") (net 2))
 (segment (start 108.17 124.583539) (end 108.17 116.88) (width 0.25) (layer "B.Cu") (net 2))
 (segment (start 109.275 136.595) (end 121.145 136.595) (width 0.25) (layer "B.Cu") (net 2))
 (segment (start 121.145 136.595) (end 123.015 138.465) (width 0.25) (layer "B.Cu") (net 2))
 (segment (start 108.15 137.72) (end 109.43 136.44) (width 0.25) (layer "B.Cu") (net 2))
 (segment (start 108.15 132.64) (end 106.07 130.56) (width 0.25) (layer "F.Cu") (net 10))
 (segment (start 105.28 134.84) (end 101.94 138.18) (width 0.25) (layer "F.Cu") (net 10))
 (segment (start 105.28 130.56) (end 105.28 134.84) (width 0.25) (layer "F.Cu") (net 10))
 (segment (start 106.07 130.56) (end 105.28 130.56) (width 0.25) (layer "F.Cu") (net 10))
 (segment (start 105.29 127.21) (end 107.44 125.06) (width 0.25) (layer "F.Cu") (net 9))
 (segment (start 107.44 125.06) (end 110.69 125.06) (width 0.25) (layer "F.Cu") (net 9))
 (segment (start 108.15 130.1) (end 107.485 129.435) (width 0.25) (layer "F.Cu") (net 9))
 (segment (start 107.485 129.435) (end 107.485 129.405) (width 0.25) (layer "F.Cu") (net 9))
 (segment (start 107.485 129.405) (end 105.29 127.21) (width 0.25) (layer "F.Cu") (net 9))
 (segment (start 101.94 130.56) (end 105.29 127.21) (width 0.25) (layer "F.Cu") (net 9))
 (segment (start 105.27 109.73) (end 105.27 114.06) (width 0.25) (layer "F.Cu") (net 16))
 (segment (start 106.1 109.73) (end 105.27 109.73) (width 0.25) (layer "F.Cu") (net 16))
 (segment (start 108.17 111.8) (end 106.1 109.73) (width 0.25) (layer "F.Cu") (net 16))
 (segment (start 105.27 114.06) (end 102 117.33) (width 0.25) (layer "F.Cu") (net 16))
 (segment (start 115.77 135.18) (end 118.77 138.18) (width 0.25) (layer "F.Cu") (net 8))
 (segment (start 118.77 138.18) (end 118.89 138.18) (width 0.25) (layer "F.Cu") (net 8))
 (segment (start 113.23 132.64) (end 115.77 135.18) (width 0.25) (layer "F.Cu") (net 8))
 (segment (start 113.23 125.06) (end 113.23 132.64) (width 0.25) (layer "F.Cu") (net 8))
 (segment (start 108.17 109.26) (end 108.16 109.26) (width 0.25) (layer "F.Cu") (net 20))
 (segment (start 108.16 109.26) (end 105.305 106.405) (width 0.25) (layer "F.Cu") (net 20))
 (segment (start 102 109.71) (end 105.305 106.405) (width 0.25) (layer "F.Cu") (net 20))
 (segment (start 107.56 104.15) (end 110.72 104.15) (width 0.25) (layer "F.Cu") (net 20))
 (segment (start 105.305 106.405) (end 107.56 104.15) (width 0.25) (layer "F.Cu") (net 20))
 (segment (start 118.65 117.2) (end 118.65 117.33) (width 0.25) (layer "F.Cu") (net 17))
 (segment (start 115.79 114.34) (end 118.65 117.2) (width 0.25) (layer "F.Cu") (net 17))
 (segment (start 113.26 104.15) (end 113.26 111.81) (width 0.25) (layer "F.Cu") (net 17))
 (segment (start 113.26 111.81) (end 115.79 114.34) (width 0.25) (layer "F.Cu") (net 17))
 (segment (start 129.83 111.76) (end 127.78 109.71) (width 0.25) (layer "F.Cu") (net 6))
 (segment (start 126.89 114.07) (end 123.64 117.32) (width 0.25) (layer "F.Cu") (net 6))
 (segment (start 126.89 109.71) (end 126.89 114.07) (width 0.25) (layer "F.Cu") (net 6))
 (segment (start 127.78 109.71) (end 126.89 109.71) (width 0.25) (layer "F.Cu") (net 6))
 (segment (start 129.22 104.12) (end 132.48 104.12) (width 0.25) (layer "F.Cu") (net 5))
 (segment (start 126.97 106.37) (end 129.22 104.12) (width 0.25) (layer "F.Cu") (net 5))
 (segment (start 123.64 109.7) (end 126.97 106.37) (width 0.25) (layer "F.Cu") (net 5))
 (segment (start 129.82 109.22) (end 126.97 106.37) (width 0.25) (layer "F.Cu") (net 5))
 (segment (start 129.83 109.22) (end 129.82 109.22) (width 0.25) (layer "F.Cu") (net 5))
 (segment (start 140.33 117.18) (end 140.33 117.36) (width 0.25) (layer "F.Cu") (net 3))
 (segment (start 135.02 111.87) (end 137.45 114.3) (width 0.25) (layer "F.Cu") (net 3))
 (segment (start 135.02 104.12) (end 135.02 111.87) (width 0.25) (layer "F.Cu") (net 3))
 (segment (start 137.45 114.3) (end 140.33 117.18) (width 0.25) (layer "F.Cu") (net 3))
 (segment (start 127.02 129.68) (end 127.02 133.94) (width 0.25) (layer "F.Cu") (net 12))
 (segment (start 129.84 131.78) (end 127.74 129.68) (width 0.25) (layer "F.Cu") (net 12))
 (segment (start 127.02 133.94) (end 123.62 137.34) (width 0.25) (layer "F.Cu") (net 12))
 (segment (start 127.74 129.68) (end 127.02 129.68) (width 0.25) (layer "F.Cu") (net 12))
 (segment (start 123.62 129.72) (end 126.93 126.41) (width 0.25) (layer "F.Cu") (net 11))
 (segment (start 126.93 126.41) (end 129.21 124.13) (width 0.25) (layer "F.Cu") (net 11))
 (segment (start 127.01 126.41) (end 126.93 126.41) (width 0.25) (layer "F.Cu") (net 11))
 (segment (start 129.84 129.24) (end 127.01 126.41) (width 0.25) (layer "F.Cu") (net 11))
 (segment (start 129.21 124.13) (end 132.44 124.13) (width 0.25) (layer "F.Cu") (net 11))
 (segment (start 140.32 137.18) (end 140.32 137.35) (width 0.25) (layer "F.Cu") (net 13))
 (segment (start 134.98 131.84) (end 137.46 134.32) (width 0.25) (layer "F.Cu") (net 13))
 (segment (start 134.98 124.13) (end 134.98 131.84) (width 0.25) (layer "F.Cu") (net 13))
 (segment (start 137.46 134.32) (end 140.32 137.18) (width 0.25) (layer "F.Cu") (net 13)))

